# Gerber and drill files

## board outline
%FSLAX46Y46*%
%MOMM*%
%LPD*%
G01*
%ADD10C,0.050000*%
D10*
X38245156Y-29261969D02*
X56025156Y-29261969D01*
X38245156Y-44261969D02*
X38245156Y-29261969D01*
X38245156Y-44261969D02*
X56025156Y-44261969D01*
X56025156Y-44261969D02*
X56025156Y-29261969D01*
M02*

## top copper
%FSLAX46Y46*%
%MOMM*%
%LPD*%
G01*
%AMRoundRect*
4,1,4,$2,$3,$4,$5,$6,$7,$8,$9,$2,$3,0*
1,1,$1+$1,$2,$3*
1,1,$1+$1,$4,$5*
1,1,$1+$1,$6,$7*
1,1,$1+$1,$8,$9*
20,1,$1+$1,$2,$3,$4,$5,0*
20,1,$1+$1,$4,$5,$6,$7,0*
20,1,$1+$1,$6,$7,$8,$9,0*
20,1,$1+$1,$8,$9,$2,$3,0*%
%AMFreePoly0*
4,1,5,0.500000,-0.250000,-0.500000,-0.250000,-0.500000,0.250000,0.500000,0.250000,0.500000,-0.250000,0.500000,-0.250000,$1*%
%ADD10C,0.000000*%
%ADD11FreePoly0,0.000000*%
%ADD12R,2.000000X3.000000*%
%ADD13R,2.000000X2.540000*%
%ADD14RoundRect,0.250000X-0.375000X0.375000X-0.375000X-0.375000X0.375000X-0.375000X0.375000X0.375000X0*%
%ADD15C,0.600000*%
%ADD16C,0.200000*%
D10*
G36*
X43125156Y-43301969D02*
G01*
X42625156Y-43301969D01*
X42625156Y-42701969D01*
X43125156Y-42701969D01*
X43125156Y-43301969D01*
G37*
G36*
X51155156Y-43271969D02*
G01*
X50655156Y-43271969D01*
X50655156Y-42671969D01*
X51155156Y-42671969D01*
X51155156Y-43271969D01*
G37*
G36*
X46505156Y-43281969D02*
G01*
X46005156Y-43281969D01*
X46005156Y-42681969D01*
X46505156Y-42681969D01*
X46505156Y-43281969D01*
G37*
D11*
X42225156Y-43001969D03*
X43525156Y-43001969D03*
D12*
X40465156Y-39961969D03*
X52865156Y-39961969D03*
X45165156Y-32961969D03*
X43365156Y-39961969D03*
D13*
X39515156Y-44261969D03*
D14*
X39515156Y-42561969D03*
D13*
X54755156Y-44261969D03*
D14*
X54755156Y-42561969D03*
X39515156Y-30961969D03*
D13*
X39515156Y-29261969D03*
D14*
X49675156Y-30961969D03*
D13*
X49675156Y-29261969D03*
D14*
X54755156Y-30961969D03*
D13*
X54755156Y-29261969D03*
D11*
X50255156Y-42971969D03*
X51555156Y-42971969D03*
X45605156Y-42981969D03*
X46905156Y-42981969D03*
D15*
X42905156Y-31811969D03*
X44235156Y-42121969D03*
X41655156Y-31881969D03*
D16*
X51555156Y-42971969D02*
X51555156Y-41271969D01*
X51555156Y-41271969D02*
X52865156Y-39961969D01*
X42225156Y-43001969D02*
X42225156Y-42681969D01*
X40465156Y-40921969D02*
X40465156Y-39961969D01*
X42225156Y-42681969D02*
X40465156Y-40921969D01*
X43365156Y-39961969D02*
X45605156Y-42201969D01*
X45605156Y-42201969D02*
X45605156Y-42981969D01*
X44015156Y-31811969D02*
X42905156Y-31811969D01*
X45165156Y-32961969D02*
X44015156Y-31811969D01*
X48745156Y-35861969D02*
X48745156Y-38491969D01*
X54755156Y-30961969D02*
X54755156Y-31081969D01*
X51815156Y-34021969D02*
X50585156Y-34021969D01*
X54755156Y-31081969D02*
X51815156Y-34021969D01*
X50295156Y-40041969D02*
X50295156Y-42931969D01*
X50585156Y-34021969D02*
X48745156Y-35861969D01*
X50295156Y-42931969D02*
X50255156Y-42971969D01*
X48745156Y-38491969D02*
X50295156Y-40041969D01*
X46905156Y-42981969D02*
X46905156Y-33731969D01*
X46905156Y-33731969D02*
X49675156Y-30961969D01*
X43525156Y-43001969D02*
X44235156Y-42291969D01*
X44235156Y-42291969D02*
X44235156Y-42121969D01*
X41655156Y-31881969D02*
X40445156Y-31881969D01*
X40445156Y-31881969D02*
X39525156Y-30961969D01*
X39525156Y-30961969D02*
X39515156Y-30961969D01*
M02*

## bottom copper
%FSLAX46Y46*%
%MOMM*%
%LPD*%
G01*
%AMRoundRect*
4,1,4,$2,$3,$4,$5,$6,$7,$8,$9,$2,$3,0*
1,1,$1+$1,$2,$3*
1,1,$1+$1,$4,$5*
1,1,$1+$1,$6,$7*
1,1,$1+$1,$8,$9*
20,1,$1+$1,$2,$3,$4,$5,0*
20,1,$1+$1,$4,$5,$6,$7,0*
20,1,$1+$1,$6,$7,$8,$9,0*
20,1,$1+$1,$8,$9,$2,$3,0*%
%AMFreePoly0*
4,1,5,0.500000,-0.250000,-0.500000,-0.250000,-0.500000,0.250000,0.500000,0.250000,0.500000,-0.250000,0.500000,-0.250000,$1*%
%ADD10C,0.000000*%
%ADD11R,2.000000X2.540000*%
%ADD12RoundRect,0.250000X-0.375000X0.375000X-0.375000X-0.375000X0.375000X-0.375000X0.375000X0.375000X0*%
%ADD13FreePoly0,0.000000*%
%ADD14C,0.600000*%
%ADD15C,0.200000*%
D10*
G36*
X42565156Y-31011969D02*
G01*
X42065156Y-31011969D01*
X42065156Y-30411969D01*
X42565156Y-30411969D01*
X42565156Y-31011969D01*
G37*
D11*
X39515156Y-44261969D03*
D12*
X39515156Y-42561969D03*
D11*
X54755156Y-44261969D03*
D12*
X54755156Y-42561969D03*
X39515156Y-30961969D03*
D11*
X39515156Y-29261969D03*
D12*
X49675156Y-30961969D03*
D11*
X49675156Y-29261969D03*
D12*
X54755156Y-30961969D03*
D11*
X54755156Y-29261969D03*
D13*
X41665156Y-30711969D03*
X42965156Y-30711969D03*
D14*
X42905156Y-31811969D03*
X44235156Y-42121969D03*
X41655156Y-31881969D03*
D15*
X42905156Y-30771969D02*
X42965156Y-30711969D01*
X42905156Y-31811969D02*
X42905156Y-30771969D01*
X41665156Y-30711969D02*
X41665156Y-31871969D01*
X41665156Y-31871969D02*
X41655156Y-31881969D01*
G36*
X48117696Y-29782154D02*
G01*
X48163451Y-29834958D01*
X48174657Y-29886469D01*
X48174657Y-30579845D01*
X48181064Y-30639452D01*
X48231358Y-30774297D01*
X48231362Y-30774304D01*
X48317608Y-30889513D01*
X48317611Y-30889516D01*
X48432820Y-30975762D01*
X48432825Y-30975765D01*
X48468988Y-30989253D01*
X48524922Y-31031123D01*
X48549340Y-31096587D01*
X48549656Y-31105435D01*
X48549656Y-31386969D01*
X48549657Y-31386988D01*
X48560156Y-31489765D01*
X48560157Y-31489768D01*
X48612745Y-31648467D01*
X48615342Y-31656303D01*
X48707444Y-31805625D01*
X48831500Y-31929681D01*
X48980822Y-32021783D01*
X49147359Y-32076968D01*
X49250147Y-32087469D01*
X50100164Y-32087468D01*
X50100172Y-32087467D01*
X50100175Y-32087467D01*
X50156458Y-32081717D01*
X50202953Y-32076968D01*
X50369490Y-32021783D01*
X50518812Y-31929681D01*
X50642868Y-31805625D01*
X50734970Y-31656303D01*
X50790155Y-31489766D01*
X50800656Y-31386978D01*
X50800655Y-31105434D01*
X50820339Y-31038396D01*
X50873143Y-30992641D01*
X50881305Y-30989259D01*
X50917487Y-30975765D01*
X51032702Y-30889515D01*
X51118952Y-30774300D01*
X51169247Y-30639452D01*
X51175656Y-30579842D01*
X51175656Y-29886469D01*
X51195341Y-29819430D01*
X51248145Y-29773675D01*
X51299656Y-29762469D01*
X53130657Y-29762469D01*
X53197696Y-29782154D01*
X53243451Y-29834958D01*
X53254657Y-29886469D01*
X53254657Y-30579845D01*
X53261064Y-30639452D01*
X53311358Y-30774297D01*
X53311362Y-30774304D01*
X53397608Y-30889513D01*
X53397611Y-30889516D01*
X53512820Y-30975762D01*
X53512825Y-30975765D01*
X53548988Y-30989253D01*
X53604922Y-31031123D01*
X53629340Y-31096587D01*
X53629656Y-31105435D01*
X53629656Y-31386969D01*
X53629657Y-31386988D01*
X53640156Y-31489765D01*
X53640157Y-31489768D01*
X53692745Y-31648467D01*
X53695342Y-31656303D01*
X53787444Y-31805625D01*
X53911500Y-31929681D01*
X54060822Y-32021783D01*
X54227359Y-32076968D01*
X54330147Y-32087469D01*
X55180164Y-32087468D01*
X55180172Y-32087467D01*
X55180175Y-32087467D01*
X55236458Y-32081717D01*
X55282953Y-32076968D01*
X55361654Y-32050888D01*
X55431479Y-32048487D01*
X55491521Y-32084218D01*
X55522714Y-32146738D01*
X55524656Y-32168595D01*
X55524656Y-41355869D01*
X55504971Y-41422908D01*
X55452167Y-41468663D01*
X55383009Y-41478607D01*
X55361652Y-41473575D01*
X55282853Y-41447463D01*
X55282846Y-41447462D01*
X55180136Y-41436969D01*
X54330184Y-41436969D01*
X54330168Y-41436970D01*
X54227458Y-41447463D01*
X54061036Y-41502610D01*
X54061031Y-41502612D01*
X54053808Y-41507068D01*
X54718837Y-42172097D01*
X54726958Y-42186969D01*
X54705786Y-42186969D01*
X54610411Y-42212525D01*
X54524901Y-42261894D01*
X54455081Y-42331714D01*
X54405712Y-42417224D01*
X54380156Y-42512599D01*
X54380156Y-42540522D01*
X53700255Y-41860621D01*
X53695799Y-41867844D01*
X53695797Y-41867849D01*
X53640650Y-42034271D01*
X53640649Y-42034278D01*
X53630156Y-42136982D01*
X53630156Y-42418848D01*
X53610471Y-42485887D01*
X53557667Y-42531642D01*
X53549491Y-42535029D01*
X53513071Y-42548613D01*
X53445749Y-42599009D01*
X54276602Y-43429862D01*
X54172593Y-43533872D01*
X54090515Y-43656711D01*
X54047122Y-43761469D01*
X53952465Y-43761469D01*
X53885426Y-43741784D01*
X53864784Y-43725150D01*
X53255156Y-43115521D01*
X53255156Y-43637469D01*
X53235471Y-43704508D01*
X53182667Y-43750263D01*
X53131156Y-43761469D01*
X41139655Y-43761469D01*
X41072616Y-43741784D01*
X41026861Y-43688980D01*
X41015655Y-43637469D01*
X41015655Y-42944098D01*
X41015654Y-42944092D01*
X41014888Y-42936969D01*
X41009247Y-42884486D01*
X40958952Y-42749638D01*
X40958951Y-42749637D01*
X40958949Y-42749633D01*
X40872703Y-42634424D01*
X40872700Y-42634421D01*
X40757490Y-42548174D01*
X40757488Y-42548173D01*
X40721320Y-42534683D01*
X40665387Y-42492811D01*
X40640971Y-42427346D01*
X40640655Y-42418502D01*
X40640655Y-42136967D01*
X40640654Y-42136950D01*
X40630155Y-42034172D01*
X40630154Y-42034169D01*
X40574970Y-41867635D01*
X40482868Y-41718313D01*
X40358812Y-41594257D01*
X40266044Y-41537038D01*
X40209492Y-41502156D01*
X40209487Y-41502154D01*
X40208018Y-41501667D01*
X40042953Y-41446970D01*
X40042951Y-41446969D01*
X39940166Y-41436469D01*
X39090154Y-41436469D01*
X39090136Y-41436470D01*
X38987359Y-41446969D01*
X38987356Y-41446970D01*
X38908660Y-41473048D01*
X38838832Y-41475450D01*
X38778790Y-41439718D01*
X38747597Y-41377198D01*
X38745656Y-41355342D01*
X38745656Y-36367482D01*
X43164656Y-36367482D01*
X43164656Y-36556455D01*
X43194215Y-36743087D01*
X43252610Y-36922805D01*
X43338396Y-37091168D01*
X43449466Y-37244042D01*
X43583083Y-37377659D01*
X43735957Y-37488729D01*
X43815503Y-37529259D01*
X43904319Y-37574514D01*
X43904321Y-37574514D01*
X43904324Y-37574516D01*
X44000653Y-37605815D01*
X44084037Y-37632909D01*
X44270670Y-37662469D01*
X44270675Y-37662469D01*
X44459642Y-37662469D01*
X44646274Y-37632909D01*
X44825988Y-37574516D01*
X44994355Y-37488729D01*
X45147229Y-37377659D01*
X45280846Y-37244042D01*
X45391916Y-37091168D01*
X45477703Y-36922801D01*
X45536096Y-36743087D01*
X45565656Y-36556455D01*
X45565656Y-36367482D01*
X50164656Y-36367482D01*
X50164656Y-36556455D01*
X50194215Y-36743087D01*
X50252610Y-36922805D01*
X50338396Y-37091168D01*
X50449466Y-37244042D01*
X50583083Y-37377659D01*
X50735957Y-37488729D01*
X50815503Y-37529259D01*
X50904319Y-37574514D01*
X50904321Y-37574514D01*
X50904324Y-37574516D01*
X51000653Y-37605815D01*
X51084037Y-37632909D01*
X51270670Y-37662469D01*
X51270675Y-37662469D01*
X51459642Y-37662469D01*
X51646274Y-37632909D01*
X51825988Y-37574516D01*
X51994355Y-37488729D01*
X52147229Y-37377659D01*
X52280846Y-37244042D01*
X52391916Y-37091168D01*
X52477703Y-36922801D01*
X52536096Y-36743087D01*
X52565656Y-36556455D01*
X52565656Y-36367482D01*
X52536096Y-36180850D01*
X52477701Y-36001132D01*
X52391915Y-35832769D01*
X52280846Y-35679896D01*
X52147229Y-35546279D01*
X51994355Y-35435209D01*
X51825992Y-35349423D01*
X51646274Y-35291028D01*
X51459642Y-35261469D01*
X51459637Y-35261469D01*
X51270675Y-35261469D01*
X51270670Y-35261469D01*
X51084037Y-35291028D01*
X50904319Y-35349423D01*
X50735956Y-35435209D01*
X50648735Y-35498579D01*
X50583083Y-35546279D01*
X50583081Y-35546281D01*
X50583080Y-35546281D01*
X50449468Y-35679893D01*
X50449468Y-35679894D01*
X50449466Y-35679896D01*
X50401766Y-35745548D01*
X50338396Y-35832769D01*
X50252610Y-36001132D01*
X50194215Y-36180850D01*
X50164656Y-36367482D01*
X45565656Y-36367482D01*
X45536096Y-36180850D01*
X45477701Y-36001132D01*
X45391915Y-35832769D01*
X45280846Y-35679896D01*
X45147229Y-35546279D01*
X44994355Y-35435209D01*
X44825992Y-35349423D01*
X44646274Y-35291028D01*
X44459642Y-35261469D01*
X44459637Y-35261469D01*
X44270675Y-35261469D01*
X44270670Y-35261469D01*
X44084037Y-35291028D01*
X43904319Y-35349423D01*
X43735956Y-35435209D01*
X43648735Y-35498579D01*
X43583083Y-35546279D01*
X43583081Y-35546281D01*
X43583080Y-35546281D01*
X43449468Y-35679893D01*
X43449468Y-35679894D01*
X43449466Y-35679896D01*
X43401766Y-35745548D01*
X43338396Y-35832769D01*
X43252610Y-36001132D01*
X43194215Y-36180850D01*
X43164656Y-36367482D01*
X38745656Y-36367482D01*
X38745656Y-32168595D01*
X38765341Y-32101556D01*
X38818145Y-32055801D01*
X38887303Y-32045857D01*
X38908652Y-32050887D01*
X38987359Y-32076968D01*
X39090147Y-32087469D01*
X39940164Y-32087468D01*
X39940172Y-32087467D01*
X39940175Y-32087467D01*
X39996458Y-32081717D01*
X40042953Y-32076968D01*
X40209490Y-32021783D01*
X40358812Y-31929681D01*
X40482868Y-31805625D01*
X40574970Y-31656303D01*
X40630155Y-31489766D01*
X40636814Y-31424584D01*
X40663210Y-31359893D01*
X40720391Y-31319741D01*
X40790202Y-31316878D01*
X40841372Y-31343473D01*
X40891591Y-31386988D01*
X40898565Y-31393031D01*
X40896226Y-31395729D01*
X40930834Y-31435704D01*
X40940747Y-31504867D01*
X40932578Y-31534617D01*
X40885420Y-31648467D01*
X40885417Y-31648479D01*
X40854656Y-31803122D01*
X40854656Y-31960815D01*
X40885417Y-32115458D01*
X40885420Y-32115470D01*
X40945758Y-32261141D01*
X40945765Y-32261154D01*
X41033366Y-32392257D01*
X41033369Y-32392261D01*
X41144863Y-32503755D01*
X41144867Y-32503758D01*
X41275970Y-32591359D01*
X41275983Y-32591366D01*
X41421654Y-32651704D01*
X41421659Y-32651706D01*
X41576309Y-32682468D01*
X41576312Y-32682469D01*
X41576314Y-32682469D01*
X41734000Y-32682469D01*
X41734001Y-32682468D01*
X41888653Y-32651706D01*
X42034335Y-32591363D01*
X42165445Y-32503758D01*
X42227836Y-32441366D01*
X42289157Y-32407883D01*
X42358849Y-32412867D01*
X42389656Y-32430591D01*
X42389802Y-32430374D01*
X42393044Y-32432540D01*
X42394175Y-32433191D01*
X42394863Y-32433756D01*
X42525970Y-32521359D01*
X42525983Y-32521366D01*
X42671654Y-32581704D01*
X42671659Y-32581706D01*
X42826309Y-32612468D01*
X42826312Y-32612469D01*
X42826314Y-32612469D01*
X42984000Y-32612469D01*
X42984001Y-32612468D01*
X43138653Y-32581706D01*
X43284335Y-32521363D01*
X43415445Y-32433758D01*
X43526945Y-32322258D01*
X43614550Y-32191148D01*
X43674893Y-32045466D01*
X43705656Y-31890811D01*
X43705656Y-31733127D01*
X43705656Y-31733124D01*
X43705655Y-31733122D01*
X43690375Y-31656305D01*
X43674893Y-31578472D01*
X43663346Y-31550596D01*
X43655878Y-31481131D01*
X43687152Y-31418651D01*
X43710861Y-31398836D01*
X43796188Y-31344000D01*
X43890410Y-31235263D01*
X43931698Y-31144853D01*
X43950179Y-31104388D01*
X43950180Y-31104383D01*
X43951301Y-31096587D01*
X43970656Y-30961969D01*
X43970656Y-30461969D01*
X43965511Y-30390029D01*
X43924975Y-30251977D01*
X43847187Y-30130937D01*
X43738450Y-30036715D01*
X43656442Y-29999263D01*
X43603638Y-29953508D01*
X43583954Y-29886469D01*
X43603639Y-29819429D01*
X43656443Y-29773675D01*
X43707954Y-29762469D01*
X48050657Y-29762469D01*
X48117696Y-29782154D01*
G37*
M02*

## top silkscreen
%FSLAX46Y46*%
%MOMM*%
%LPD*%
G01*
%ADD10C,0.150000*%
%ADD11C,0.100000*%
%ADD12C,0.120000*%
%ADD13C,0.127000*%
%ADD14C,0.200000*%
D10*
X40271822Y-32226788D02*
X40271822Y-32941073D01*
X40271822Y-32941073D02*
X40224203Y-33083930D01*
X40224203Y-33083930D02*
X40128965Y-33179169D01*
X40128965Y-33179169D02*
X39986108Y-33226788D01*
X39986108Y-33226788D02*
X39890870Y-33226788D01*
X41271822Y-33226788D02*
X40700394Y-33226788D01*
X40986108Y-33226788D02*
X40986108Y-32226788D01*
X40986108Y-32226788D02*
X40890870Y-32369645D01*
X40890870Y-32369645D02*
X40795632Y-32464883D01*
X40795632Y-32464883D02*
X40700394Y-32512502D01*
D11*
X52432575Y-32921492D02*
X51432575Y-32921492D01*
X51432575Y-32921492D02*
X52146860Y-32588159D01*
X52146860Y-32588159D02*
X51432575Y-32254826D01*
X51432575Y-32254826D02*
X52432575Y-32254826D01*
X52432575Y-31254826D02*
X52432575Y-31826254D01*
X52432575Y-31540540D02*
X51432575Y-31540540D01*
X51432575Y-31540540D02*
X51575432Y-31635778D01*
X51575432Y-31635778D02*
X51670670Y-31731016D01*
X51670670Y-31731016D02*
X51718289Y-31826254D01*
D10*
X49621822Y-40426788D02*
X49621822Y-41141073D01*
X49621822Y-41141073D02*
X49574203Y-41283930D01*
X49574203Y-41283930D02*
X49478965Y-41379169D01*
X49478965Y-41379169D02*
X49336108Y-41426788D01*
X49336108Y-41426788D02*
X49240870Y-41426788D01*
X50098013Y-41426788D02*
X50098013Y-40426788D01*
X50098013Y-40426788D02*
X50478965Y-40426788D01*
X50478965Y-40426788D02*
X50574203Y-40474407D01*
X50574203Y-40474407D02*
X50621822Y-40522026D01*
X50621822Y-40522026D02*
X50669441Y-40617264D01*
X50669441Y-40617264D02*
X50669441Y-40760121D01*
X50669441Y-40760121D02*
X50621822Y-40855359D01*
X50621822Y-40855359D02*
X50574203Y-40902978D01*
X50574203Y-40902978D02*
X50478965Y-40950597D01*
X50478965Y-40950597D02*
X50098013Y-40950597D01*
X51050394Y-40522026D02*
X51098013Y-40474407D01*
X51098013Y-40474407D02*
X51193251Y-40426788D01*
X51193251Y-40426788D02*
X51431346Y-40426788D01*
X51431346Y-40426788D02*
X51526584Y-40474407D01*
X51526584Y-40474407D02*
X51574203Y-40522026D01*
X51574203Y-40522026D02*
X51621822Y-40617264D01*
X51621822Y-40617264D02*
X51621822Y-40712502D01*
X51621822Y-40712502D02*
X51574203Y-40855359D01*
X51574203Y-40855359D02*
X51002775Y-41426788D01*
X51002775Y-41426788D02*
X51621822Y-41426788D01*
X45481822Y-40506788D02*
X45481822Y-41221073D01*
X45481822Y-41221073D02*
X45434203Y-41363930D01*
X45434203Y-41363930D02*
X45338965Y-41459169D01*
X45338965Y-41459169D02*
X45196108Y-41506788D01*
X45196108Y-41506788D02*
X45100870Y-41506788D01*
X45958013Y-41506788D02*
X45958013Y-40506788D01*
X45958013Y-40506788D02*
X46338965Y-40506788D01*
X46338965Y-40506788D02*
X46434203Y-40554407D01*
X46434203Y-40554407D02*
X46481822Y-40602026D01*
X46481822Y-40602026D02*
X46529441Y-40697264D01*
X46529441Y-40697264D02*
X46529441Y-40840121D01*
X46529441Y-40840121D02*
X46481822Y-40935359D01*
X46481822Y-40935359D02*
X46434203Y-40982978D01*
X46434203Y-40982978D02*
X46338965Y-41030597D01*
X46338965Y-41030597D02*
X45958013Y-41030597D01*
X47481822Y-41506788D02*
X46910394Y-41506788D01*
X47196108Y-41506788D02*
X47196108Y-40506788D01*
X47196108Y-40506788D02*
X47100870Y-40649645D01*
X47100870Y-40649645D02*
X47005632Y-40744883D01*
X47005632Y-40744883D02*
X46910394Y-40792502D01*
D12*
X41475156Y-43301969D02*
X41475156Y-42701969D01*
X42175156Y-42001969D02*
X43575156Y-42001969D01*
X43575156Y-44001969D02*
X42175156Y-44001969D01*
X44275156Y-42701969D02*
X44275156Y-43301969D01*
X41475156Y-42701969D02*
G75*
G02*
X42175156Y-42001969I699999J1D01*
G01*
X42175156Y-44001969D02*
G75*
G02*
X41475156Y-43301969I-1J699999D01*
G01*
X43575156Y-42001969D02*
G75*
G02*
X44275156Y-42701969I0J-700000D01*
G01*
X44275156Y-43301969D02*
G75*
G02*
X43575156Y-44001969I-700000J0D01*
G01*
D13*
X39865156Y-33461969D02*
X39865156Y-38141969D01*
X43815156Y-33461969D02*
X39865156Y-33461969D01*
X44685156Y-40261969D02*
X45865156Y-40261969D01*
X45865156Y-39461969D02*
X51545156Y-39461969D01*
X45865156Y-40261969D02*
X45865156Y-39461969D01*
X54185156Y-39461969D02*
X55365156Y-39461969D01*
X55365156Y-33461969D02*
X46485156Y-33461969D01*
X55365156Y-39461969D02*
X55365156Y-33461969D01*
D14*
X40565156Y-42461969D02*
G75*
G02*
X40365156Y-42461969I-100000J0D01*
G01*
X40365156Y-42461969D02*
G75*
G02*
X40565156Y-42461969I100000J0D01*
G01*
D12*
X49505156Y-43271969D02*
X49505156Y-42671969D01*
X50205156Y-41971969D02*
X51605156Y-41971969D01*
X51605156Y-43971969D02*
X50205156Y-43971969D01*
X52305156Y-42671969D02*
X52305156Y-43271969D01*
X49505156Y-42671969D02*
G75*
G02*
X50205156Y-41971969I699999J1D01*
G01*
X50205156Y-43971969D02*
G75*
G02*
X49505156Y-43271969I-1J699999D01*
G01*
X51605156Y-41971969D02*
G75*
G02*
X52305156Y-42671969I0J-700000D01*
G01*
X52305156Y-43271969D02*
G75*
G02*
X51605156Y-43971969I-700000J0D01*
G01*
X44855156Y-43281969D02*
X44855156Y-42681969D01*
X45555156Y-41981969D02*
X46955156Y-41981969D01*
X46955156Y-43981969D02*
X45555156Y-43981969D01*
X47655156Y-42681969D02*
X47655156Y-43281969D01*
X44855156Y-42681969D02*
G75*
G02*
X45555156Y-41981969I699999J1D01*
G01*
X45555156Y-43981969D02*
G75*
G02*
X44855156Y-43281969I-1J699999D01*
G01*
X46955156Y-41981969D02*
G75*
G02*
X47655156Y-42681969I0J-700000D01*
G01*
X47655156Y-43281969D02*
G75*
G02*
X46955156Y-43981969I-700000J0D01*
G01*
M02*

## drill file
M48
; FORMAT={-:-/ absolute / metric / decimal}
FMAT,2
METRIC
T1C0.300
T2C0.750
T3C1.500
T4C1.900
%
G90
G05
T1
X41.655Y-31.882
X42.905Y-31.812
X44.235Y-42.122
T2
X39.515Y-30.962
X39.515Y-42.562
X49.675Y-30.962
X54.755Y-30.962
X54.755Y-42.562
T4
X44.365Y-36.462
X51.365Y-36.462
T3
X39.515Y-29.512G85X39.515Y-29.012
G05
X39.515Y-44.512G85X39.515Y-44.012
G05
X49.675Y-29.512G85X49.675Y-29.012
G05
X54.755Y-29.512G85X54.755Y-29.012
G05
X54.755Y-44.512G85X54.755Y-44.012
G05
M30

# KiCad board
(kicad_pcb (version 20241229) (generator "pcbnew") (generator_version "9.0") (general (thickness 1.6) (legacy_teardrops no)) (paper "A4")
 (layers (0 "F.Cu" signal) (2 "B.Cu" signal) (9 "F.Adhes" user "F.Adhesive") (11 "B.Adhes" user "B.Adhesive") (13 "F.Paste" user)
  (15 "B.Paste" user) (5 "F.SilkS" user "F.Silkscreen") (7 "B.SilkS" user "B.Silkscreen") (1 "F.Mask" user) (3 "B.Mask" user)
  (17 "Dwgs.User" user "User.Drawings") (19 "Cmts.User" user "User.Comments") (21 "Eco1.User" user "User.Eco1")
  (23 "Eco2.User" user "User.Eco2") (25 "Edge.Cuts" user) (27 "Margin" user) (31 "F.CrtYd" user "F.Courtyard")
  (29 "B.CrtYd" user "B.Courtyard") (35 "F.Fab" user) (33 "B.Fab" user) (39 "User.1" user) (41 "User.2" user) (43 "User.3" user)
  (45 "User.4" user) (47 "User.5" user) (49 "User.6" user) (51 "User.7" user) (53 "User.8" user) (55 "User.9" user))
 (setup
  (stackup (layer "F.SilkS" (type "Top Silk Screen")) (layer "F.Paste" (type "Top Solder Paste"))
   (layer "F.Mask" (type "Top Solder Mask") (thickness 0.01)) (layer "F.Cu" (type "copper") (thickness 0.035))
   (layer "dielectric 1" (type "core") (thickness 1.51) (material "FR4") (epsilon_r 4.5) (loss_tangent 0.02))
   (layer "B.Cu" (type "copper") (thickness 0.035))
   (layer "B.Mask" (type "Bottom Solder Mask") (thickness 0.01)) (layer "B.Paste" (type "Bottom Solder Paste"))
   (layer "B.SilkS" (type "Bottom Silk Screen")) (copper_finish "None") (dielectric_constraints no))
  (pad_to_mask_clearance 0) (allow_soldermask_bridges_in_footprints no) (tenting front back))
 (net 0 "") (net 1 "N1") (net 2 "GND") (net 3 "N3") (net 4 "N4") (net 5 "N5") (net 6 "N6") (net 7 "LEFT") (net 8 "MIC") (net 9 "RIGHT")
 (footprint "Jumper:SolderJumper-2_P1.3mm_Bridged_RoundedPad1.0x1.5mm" (layer "F.Cu") (at 42.875156 43.001969)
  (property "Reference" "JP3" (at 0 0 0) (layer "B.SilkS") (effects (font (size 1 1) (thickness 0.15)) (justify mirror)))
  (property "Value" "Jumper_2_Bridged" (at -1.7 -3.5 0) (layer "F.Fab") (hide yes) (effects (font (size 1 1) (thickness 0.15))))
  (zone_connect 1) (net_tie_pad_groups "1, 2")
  (fp_poly (pts (xy 0.25 -0.3) (xy -0.25 -0.3) (xy -0.25 0.3) (xy 0.25 0.3)) (stroke (width 0) (type solid)) (fill yes) (layer "F.Cu"))
  (fp_line (start -1.4 0.3) (end -1.4 -0.3) (stroke (width 0.12) (type solid)) (layer "F.SilkS"))
  (fp_line (start -0.7 -1) (end 0.7 -1) (stroke (width 0.12) (type solid)) (layer "F.SilkS"))
  (fp_line (start 0.7 1) (end -0.7 1) (stroke (width 0.12) (type solid)) (layer "F.SilkS"))
  (fp_line (start 1.4 -0.3) (end 1.4 0.3) (stroke (width 0.12) (type solid)) (layer "F.SilkS"))
  (fp_arc (start -1.4 -0.3) (mid -1.194975 -0.794975) (end -0.7 -1) (stroke (width 0.12) (type solid)) (layer "F.SilkS"))
  (fp_arc (start -0.7 1) (mid -1.194975 0.794975) (end -1.4 0.3) (stroke (width 0.12) (type solid)) (layer "F.SilkS"))
  (fp_arc (start 0.7 -1) (mid 1.194975 -0.794975) (end 1.4 -0.3) (stroke (width 0.12) (type solid)) (layer "F.SilkS"))
  (fp_arc (start 1.4 0.3) (mid 1.194975 0.794975) (end 0.7 1) (stroke (width 0.12) (type solid)) (layer "F.SilkS"))
  (pad "1" smd custom (at -0.65 0) (size 1 0.5) (layers "F.Cu" "F.Mask") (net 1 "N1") (zone_connect 2) (thermal_bridge_angle 45)
   (options (clearance outline) (anchor rect)) (primitives))
  (pad "2" smd custom (at 0.65 0) (size 1 0.5) (layers "F.Cu" "F.Mask") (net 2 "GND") (zone_connect 2) (thermal_bridge_angle 45)
   (options (clearance outline) (anchor rect)) (primitives)))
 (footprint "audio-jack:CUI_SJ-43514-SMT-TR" (layer "F.Cu") (at 40.465156 39.961969)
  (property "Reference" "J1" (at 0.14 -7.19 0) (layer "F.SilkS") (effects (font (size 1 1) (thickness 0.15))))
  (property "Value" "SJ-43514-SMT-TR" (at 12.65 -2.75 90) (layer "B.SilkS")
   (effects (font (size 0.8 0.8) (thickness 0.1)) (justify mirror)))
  (fp_line (start -0.6 -6.5) (end -0.6 -1.82) (stroke (width 0.127) (type solid)) (layer "F.SilkS"))
  (fp_line (start 3.35 -6.5) (end -0.6 -6.5) (stroke (width 0.127) (type solid)) (layer "F.SilkS"))
  (fp_line (start 4.22 0.3) (end 5.4 0.3) (stroke (width 0.127) (type solid)) (layer "F.SilkS"))
  (fp_line (start 5.4 -0.5) (end 11.08 -0.5) (stroke (width 0.127) (type solid)) (layer "F.SilkS"))
  (fp_line (start 5.4 0.3) (end 5.4 -0.5) (stroke (width 0.127) (type solid)) (layer "F.SilkS"))
  (fp_line (start 13.72 -0.5) (end 14.9 -0.5) (stroke (width 0.127) (type solid)) (layer "F.SilkS"))
  (fp_line (start 14.9 -6.5) (end 6.02 -6.5) (stroke (width 0.127) (type solid)) (layer "F.SilkS"))
  (fp_line (start 14.9 -0.5) (end 14.9 -6.5) (stroke (width 0.127) (type solid)) (layer "F.SilkS"))
  (fp_circle (center 0 2.5) (end 0.1 2.5) (stroke (width 0.2) (type solid)) (fill no) (layer "F.SilkS"))
  (pad "" np_thru_hole circle (at 3.9 -3.5) (size 1.9 1.9) (drill 1.9) (layers "*.Cu" "*.Mask"))
  (pad "" np_thru_hole circle (at 10.9 -3.5) (size 1.9 1.9) (drill 1.9) (layers "*.Cu" "*.Mask"))
  (pad "1" smd rect (at 0 0) (size 2 3) (layers "F.Cu" "F.Mask" "F.Paste") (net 1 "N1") (solder_mask_margin 0.102))
  (pad "2" smd rect (at 12.4 0) (size 2 3) (layers "F.Cu" "F.Mask" "F.Paste") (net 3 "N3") (solder_mask_margin 0.102))
  (pad "3" smd rect (at 4.7 -7) (size 2 3) (layers "F.Cu" "F.Mask" "F.Paste") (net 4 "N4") (solder_mask_margin 0.102))
  (pad "4" smd rect (at 2.9 0) (size 2 3) (layers "F.Cu" "F.Mask" "F.Paste") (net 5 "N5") (solder_mask_margin 0.102)))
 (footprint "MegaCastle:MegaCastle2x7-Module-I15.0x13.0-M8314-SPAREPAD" (layer "F.Cu") (at 47.135156 36.761969 90)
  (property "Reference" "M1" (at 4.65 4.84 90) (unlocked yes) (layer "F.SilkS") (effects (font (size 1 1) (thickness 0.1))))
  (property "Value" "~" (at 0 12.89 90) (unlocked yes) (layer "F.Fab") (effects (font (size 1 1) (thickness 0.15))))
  (fp_line (start 7.5 -8.89) (end 7.5 8.89) (stroke (width 0.05) (type default)) (layer "Edge.Cuts"))
  (fp_line (start -7.5 -8.89) (end 7.5 -8.89) (stroke (width 0.05) (type default)) (layer "Edge.Cuts"))
  (fp_line (start -7.5 -8.89) (end -7.5 8.89) (stroke (width 0.05) (type default)) (layer "Edge.Cuts"))
  (fp_line (start -7.5 8.89) (end 7.5 8.89) (stroke (width 0.05) (type default)) (layer "Edge.Cuts"))
  (pad "1" thru_hole rect (at -7.5 -7.62 90) (size 2.54 2) (drill oval 2 1.5) (layers "*.Cu" "*.Mask") (remove_unused_layers no)
   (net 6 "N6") (thermal_bridge_angle 45))
  (pad "1" thru_hole roundrect (at -5.8 -7.62 270) (size 1.25 1.25) (drill 0.75) (layers "*.Cu" "*.Mask") (remove_unused_layers no)
   (roundrect_rratio 0.2) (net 6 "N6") (thermal_bridge_angle 45))
  (pad "7" thru_hole rect (at -7.5 7.62 90) (size 2.54 2) (drill oval 2 1.5) (layers "*.Cu" "*.Mask") (remove_unused_layers no)
   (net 2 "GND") (thermal_bridge_angle 45))
  (pad "7" thru_hole roundrect (at -5.8 7.62 270) (size 1.25 1.25) (drill 0.75) (layers "*.Cu" "*.Mask") (remove_unused_layers no)
   (roundrect_rratio 0.2) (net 2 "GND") (thermal_bridge_angle 45))
  (pad "8" thru_hole roundrect (at 5.8 -7.62 270) (size 1.25 1.25) (drill 0.75) (layers "*.Cu" "*.Mask") (remove_unused_layers no)
   (roundrect_rratio 0.2) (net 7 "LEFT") (thermal_bridge_angle 45))
  (pad "8" thru_hole rect (at 7.5 -7.62 90) (size 2.54 2) (drill oval 2 1.5) (layers "*.Cu" "*.Mask") (remove_unused_layers no)
   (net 7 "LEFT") (thermal_bridge_angle 45))
  (pad "12" thru_hole roundrect (at 5.8 2.54 270) (size 1.25 1.25) (drill 0.75) (layers "*.Cu" "*.Mask") (remove_unused_layers no)
   (roundrect_rratio 0.2) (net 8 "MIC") (thermal_bridge_angle 45))
  (pad "12" thru_hole rect (at 7.5 2.54 90) (size 2.54 2) (drill oval 2 1.5) (layers "*.Cu" "*.Mask") (remove_unused_layers no)
   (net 8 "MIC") (thermal_bridge_angle 45))
  (pad "14" thru_hole roundrect (at 5.8 7.62 270) (size 1.25 1.25) (drill 0.75) (layers "*.Cu" "*.Mask") (remove_unused_layers no)
   (roundrect_rratio 0.2) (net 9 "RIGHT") (thermal_bridge_angle 45))
  (pad "14" thru_hole rect (at 7.5 7.62 90) (size 2.54 2) (drill oval 2 1.5) (layers "*.Cu" "*.Mask") (remove_unused_layers no)
   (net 9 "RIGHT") (thermal_bridge_angle 45))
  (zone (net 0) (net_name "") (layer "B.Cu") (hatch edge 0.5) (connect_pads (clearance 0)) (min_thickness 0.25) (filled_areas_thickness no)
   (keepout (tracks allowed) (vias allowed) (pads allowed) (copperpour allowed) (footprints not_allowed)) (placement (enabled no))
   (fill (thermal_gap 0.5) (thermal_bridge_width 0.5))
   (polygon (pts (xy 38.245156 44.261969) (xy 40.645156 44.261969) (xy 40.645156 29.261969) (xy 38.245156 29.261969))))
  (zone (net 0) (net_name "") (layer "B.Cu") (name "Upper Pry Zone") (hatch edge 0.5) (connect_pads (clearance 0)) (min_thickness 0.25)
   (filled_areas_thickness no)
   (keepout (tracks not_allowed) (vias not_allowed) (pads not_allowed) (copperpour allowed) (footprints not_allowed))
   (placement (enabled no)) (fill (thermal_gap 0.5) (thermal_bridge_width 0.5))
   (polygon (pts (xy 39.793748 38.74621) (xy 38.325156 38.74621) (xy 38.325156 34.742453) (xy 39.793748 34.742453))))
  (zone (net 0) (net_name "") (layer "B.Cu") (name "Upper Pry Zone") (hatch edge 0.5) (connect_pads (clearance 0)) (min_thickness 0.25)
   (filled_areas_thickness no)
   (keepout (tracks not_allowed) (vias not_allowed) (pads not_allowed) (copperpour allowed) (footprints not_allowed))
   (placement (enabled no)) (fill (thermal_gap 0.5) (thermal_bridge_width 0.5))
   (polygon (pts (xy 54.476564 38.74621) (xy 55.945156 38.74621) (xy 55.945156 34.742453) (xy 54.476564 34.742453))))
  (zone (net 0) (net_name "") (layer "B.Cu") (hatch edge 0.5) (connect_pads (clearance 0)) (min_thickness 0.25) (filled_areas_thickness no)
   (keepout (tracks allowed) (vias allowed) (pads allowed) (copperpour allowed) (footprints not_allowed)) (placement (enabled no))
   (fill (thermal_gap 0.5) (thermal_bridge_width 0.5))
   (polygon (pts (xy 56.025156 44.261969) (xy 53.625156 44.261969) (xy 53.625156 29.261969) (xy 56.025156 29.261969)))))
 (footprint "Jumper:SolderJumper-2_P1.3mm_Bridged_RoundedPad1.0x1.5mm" (layer "F.Cu") (at 50.905156 42.971969)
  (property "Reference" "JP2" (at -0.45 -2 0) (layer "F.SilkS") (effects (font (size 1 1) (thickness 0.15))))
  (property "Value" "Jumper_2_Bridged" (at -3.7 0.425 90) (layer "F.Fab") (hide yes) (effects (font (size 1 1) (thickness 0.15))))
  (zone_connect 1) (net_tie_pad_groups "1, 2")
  (fp_poly (pts (xy 0.25 -0.3) (xy -0.25 -0.3) (xy -0.25 0.3) (xy 0.25 0.3)) (stroke (width 0) (type solid)) (fill yes) (layer "F.Cu"))
  (fp_line (start -1.4 0.3) (end -1.4 -0.3) (stroke (width 0.12) (type solid)) (layer "F.SilkS"))
  (fp_line (start -0.7 -1) (end 0.7 -1) (stroke (width 0.12) (type solid)) (layer "F.SilkS"))
  (fp_line (start 0.7 1) (end -0.7 1) (stroke (width 0.12) (type solid)) (layer "F.SilkS"))
  (fp_line (start 1.4 -0.3) (end 1.4 0.3) (stroke (width 0.12) (type solid)) (layer "F.SilkS"))
  (fp_arc (start -1.4 -0.3) (mid -1.194975 -0.794975) (end -0.7 -1) (stroke (width 0.12) (type solid)) (layer "F.SilkS"))
  (fp_arc (start -0.7 1) (mid -1.194975 0.794975) (end -1.4 0.3) (stroke (width 0.12) (type solid)) (layer "F.SilkS"))
  (fp_arc (start 0.7 -1) (mid 1.194975 -0.794975) (end 1.4 -0.3) (stroke (width 0.12) (type solid)) (layer "F.SilkS"))
  (fp_arc (start 1.4 0.3) (mid 1.194975 0.794975) (end 0.7 1) (stroke (width 0.12) (type solid)) (layer "F.SilkS"))
  (pad "1" smd custom (at -0.65 0) (size 1 0.5) (layers "F.Cu" "F.Mask") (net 9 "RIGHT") (zone_connect 2) (thermal_bridge_angle 45)
   (options (clearance outline) (anchor rect)) (primitives))
  (pad "2" smd custom (at 0.65 0) (size 1 0.5) (layers "F.Cu" "F.Mask") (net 3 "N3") (zone_connect 2) (thermal_bridge_angle 45)
   (options (clearance outline) (anchor rect)) (primitives)))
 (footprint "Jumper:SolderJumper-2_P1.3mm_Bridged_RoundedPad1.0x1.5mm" (layer "F.Cu") (at 46.255156 42.981969)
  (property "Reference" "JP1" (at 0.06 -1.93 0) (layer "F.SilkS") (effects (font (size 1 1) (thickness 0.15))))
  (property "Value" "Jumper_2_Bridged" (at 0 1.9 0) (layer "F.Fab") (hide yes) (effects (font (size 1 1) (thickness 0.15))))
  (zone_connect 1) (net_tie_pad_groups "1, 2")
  (fp_poly (pts (xy 0.25 -0.3) (xy -0.25 -0.3) (xy -0.25 0.3) (xy 0.25 0.3)) (stroke (width 0) (type solid)) (fill yes) (layer "F.Cu"))
  (fp_line (start -1.4 0.3) (end -1.4 -0.3) (stroke (width 0.12) (type solid)) (layer "F.SilkS"))
  (fp_line (start -0.7 -1) (end 0.7 -1) (stroke (width 0.12) (type solid)) (layer "F.SilkS"))
  (fp_line (start 0.7 1) (end -0.7 1) (stroke (width 0.12) (type solid)) (layer "F.SilkS"))
  (fp_line (start 1.4 -0.3) (end 1.4 0.3) (stroke (width 0.12) (type solid)) (layer "F.SilkS"))
  (fp_arc (start -1.4 -0.3) (mid -1.194975 -0.794975) (end -0.7 -1) (stroke (width 0.12) (type solid)) (layer "F.SilkS"))
  (fp_arc (start -0.7 1) (mid -1.194975 0.794975) (end -1.4 0.3) (stroke (width 0.12) (type solid)) (layer "F.SilkS"))
  (fp_arc (start 0.7 -1) (mid 1.194975 -0.794975) (end 1.4 -0.3) (stroke (width 0.12) (type solid)) (layer "F.SilkS"))
  (fp_arc (start 1.4 0.3) (mid 1.194975 0.794975) (end 0.7 1) (stroke (width 0.12) (type solid)) (layer "F.SilkS"))
  (pad "1" smd custom (at -0.65 0) (size 1 0.5) (layers "F.Cu" "F.Mask") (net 5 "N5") (zone_connect 2) (thermal_bridge_angle 45)
   (options (clearance outline) (anchor rect)) (primitives))
  (pad "2" smd custom (at 0.65 0) (size 1 0.5) (layers "F.Cu" "F.Mask") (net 8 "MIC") (zone_connect 2) (thermal_bridge_angle 45)
   (options (clearance outline) (anchor rect)) (primitives)))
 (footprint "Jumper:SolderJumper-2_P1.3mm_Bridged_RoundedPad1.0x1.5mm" (layer "B.Cu") (at 42.315156 30.711969)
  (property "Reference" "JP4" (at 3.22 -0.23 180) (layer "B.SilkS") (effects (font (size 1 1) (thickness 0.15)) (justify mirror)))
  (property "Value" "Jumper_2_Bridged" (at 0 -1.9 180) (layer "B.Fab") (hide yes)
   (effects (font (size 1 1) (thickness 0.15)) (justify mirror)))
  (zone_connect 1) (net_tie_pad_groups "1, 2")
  (fp_poly (pts (xy 0.25 0.3) (xy -0.25 0.3) (xy -0.25 -0.3) (xy 0.25 -0.3)) (stroke (width 0) (type solid)) (fill yes) (layer "B.Cu"))
  (pad "1" smd custom (at -0.65 0) (size 1 0.5) (layers "B.Cu" "B.Mask") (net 7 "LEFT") (zone_connect 2) (thermal_bridge_angle 45)
   (options (clearance outline) (anchor rect)) (primitives))
  (pad "2" smd custom (at 0.65 0) (size 1 0.5) (layers "B.Cu" "B.Mask") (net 4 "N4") (zone_connect 2) (thermal_bridge_angle 45)
   (options (clearance outline) (anchor rect)) (primitives)))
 (segment (start 51.555156 42.971969) (end 51.555156 41.271969) (width 0.2) (layer "F.Cu") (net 3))
 (segment (start 51.555156 41.271969) (end 52.865156 39.961969) (width 0.2) (layer "F.Cu") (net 3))
 (segment (start 42.225156 43.001969) (end 42.225156 42.681969) (width 0.2) (layer "F.Cu") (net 1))
 (segment (start 40.465156 40.921969) (end 40.465156 39.961969) (width 0.2) (layer "F.Cu") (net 1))
 (segment (start 42.225156 42.681969) (end 40.465156 40.921969) (width 0.2) (layer "F.Cu") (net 1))
 (segment (start 43.365156 39.961969) (end 45.605156 42.201969) (width 0.2) (layer "F.Cu") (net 5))
 (segment (start 45.605156 42.201969) (end 45.605156 42.981969) (width 0.2) (layer "F.Cu") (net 5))
 (segment (start 44.015156 31.811969) (end 42.905156 31.811969) (width 0.2) (layer "F.Cu") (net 4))
 (segment (start 45.165156 32.961969) (end 44.015156 31.811969) (width 0.2) (layer "F.Cu") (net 4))
 (via (at 42.905156 31.811969) (size 0.6) (drill 0.3) (layers "F.Cu" "B.Cu") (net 4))
 (segment (start 42.905156 30.771969) (end 42.965156 30.711969) (width 0.2) (layer "B.Cu") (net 4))
 (segment (start 42.905156 31.811969) (end 42.905156 30.771969) (width 0.2) (layer "B.Cu") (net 4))
 (segment (start 48.745156 35.861969) (end 48.745156 38.491969) (width 0.2) (layer "F.Cu") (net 9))
 (segment (start 54.755156 30.961969) (end 54.755156 31.081969) (width 0.2) (layer "F.Cu") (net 9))
 (segment (start 51.815156 34.021969) (end 50.585156 34.021969) (width 0.2) (layer "F.Cu") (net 9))
 (segment (start 54.755156 31.081969) (end 51.815156 34.021969) (width 0.2) (layer "F.Cu") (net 9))
 (segment (start 50.295156 40.041969) (end 50.295156 42.931969) (width 0.2) (layer "F.Cu") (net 9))
 (segment (start 50.585156 34.021969) (end 48.745156 35.861969) (width 0.2) (layer "F.Cu") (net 9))
 (segment (start 50.295156 42.931969) (end 50.255156 42.971969) (width 0.2) (layer "F.Cu") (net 9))
 (segment (start 48.745156 38.491969) (end 50.295156 40.041969) (width 0.2) (layer "F.Cu") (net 9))
 (segment (start 46.905156 42.981969) (end 46.905156 33.731969) (width 0.2) (layer "F.Cu") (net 8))
 (segment (start 46.905156 33.731969) (end 49.675156 30.961969) (width 0.2) (layer "F.Cu") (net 8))
 (segment (start 43.525156 43.001969) (end 44.235156 42.291969) (width 0.2) (layer "F.Cu") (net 2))
 (segment (start 44.235156 42.291969) (end 44.235156 42.121969) (width 0.2) (layer "F.Cu") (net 2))
 (via (at 44.235156 42.121969) (size 0.6) (drill 0.3) (layers "F.Cu" "B.Cu") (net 2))
 (segment (start 41.655156 31.881969) (end 40.445156 31.881969) (width 0.2) (layer "F.Cu") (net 7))
 (segment (start 40.445156 31.881969) (end 39.525156 30.961969) (width 0.2) (layer "F.Cu") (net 7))
 (segment (start 39.525156 30.961969) (end 39.515156 30.961969) (width 0.2) (layer "F.Cu") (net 7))
 (via (at 41.655156 31.881969) (size 0.6) (drill 0.3) (layers "F.Cu" "B.Cu") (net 7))
 (segment (start 41.665156 30.711969) (end 41.665156 31.871969) (width 0.2) (layer "B.Cu") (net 7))
 (segment (start 41.665156 31.871969) (end 41.655156 31.881969) (width 0.2) (layer "B.Cu") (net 7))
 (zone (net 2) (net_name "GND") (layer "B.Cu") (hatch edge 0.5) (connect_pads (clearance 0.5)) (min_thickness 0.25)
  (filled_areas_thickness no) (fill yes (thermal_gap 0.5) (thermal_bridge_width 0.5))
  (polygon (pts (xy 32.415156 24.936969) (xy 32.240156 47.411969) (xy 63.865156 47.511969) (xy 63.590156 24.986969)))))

